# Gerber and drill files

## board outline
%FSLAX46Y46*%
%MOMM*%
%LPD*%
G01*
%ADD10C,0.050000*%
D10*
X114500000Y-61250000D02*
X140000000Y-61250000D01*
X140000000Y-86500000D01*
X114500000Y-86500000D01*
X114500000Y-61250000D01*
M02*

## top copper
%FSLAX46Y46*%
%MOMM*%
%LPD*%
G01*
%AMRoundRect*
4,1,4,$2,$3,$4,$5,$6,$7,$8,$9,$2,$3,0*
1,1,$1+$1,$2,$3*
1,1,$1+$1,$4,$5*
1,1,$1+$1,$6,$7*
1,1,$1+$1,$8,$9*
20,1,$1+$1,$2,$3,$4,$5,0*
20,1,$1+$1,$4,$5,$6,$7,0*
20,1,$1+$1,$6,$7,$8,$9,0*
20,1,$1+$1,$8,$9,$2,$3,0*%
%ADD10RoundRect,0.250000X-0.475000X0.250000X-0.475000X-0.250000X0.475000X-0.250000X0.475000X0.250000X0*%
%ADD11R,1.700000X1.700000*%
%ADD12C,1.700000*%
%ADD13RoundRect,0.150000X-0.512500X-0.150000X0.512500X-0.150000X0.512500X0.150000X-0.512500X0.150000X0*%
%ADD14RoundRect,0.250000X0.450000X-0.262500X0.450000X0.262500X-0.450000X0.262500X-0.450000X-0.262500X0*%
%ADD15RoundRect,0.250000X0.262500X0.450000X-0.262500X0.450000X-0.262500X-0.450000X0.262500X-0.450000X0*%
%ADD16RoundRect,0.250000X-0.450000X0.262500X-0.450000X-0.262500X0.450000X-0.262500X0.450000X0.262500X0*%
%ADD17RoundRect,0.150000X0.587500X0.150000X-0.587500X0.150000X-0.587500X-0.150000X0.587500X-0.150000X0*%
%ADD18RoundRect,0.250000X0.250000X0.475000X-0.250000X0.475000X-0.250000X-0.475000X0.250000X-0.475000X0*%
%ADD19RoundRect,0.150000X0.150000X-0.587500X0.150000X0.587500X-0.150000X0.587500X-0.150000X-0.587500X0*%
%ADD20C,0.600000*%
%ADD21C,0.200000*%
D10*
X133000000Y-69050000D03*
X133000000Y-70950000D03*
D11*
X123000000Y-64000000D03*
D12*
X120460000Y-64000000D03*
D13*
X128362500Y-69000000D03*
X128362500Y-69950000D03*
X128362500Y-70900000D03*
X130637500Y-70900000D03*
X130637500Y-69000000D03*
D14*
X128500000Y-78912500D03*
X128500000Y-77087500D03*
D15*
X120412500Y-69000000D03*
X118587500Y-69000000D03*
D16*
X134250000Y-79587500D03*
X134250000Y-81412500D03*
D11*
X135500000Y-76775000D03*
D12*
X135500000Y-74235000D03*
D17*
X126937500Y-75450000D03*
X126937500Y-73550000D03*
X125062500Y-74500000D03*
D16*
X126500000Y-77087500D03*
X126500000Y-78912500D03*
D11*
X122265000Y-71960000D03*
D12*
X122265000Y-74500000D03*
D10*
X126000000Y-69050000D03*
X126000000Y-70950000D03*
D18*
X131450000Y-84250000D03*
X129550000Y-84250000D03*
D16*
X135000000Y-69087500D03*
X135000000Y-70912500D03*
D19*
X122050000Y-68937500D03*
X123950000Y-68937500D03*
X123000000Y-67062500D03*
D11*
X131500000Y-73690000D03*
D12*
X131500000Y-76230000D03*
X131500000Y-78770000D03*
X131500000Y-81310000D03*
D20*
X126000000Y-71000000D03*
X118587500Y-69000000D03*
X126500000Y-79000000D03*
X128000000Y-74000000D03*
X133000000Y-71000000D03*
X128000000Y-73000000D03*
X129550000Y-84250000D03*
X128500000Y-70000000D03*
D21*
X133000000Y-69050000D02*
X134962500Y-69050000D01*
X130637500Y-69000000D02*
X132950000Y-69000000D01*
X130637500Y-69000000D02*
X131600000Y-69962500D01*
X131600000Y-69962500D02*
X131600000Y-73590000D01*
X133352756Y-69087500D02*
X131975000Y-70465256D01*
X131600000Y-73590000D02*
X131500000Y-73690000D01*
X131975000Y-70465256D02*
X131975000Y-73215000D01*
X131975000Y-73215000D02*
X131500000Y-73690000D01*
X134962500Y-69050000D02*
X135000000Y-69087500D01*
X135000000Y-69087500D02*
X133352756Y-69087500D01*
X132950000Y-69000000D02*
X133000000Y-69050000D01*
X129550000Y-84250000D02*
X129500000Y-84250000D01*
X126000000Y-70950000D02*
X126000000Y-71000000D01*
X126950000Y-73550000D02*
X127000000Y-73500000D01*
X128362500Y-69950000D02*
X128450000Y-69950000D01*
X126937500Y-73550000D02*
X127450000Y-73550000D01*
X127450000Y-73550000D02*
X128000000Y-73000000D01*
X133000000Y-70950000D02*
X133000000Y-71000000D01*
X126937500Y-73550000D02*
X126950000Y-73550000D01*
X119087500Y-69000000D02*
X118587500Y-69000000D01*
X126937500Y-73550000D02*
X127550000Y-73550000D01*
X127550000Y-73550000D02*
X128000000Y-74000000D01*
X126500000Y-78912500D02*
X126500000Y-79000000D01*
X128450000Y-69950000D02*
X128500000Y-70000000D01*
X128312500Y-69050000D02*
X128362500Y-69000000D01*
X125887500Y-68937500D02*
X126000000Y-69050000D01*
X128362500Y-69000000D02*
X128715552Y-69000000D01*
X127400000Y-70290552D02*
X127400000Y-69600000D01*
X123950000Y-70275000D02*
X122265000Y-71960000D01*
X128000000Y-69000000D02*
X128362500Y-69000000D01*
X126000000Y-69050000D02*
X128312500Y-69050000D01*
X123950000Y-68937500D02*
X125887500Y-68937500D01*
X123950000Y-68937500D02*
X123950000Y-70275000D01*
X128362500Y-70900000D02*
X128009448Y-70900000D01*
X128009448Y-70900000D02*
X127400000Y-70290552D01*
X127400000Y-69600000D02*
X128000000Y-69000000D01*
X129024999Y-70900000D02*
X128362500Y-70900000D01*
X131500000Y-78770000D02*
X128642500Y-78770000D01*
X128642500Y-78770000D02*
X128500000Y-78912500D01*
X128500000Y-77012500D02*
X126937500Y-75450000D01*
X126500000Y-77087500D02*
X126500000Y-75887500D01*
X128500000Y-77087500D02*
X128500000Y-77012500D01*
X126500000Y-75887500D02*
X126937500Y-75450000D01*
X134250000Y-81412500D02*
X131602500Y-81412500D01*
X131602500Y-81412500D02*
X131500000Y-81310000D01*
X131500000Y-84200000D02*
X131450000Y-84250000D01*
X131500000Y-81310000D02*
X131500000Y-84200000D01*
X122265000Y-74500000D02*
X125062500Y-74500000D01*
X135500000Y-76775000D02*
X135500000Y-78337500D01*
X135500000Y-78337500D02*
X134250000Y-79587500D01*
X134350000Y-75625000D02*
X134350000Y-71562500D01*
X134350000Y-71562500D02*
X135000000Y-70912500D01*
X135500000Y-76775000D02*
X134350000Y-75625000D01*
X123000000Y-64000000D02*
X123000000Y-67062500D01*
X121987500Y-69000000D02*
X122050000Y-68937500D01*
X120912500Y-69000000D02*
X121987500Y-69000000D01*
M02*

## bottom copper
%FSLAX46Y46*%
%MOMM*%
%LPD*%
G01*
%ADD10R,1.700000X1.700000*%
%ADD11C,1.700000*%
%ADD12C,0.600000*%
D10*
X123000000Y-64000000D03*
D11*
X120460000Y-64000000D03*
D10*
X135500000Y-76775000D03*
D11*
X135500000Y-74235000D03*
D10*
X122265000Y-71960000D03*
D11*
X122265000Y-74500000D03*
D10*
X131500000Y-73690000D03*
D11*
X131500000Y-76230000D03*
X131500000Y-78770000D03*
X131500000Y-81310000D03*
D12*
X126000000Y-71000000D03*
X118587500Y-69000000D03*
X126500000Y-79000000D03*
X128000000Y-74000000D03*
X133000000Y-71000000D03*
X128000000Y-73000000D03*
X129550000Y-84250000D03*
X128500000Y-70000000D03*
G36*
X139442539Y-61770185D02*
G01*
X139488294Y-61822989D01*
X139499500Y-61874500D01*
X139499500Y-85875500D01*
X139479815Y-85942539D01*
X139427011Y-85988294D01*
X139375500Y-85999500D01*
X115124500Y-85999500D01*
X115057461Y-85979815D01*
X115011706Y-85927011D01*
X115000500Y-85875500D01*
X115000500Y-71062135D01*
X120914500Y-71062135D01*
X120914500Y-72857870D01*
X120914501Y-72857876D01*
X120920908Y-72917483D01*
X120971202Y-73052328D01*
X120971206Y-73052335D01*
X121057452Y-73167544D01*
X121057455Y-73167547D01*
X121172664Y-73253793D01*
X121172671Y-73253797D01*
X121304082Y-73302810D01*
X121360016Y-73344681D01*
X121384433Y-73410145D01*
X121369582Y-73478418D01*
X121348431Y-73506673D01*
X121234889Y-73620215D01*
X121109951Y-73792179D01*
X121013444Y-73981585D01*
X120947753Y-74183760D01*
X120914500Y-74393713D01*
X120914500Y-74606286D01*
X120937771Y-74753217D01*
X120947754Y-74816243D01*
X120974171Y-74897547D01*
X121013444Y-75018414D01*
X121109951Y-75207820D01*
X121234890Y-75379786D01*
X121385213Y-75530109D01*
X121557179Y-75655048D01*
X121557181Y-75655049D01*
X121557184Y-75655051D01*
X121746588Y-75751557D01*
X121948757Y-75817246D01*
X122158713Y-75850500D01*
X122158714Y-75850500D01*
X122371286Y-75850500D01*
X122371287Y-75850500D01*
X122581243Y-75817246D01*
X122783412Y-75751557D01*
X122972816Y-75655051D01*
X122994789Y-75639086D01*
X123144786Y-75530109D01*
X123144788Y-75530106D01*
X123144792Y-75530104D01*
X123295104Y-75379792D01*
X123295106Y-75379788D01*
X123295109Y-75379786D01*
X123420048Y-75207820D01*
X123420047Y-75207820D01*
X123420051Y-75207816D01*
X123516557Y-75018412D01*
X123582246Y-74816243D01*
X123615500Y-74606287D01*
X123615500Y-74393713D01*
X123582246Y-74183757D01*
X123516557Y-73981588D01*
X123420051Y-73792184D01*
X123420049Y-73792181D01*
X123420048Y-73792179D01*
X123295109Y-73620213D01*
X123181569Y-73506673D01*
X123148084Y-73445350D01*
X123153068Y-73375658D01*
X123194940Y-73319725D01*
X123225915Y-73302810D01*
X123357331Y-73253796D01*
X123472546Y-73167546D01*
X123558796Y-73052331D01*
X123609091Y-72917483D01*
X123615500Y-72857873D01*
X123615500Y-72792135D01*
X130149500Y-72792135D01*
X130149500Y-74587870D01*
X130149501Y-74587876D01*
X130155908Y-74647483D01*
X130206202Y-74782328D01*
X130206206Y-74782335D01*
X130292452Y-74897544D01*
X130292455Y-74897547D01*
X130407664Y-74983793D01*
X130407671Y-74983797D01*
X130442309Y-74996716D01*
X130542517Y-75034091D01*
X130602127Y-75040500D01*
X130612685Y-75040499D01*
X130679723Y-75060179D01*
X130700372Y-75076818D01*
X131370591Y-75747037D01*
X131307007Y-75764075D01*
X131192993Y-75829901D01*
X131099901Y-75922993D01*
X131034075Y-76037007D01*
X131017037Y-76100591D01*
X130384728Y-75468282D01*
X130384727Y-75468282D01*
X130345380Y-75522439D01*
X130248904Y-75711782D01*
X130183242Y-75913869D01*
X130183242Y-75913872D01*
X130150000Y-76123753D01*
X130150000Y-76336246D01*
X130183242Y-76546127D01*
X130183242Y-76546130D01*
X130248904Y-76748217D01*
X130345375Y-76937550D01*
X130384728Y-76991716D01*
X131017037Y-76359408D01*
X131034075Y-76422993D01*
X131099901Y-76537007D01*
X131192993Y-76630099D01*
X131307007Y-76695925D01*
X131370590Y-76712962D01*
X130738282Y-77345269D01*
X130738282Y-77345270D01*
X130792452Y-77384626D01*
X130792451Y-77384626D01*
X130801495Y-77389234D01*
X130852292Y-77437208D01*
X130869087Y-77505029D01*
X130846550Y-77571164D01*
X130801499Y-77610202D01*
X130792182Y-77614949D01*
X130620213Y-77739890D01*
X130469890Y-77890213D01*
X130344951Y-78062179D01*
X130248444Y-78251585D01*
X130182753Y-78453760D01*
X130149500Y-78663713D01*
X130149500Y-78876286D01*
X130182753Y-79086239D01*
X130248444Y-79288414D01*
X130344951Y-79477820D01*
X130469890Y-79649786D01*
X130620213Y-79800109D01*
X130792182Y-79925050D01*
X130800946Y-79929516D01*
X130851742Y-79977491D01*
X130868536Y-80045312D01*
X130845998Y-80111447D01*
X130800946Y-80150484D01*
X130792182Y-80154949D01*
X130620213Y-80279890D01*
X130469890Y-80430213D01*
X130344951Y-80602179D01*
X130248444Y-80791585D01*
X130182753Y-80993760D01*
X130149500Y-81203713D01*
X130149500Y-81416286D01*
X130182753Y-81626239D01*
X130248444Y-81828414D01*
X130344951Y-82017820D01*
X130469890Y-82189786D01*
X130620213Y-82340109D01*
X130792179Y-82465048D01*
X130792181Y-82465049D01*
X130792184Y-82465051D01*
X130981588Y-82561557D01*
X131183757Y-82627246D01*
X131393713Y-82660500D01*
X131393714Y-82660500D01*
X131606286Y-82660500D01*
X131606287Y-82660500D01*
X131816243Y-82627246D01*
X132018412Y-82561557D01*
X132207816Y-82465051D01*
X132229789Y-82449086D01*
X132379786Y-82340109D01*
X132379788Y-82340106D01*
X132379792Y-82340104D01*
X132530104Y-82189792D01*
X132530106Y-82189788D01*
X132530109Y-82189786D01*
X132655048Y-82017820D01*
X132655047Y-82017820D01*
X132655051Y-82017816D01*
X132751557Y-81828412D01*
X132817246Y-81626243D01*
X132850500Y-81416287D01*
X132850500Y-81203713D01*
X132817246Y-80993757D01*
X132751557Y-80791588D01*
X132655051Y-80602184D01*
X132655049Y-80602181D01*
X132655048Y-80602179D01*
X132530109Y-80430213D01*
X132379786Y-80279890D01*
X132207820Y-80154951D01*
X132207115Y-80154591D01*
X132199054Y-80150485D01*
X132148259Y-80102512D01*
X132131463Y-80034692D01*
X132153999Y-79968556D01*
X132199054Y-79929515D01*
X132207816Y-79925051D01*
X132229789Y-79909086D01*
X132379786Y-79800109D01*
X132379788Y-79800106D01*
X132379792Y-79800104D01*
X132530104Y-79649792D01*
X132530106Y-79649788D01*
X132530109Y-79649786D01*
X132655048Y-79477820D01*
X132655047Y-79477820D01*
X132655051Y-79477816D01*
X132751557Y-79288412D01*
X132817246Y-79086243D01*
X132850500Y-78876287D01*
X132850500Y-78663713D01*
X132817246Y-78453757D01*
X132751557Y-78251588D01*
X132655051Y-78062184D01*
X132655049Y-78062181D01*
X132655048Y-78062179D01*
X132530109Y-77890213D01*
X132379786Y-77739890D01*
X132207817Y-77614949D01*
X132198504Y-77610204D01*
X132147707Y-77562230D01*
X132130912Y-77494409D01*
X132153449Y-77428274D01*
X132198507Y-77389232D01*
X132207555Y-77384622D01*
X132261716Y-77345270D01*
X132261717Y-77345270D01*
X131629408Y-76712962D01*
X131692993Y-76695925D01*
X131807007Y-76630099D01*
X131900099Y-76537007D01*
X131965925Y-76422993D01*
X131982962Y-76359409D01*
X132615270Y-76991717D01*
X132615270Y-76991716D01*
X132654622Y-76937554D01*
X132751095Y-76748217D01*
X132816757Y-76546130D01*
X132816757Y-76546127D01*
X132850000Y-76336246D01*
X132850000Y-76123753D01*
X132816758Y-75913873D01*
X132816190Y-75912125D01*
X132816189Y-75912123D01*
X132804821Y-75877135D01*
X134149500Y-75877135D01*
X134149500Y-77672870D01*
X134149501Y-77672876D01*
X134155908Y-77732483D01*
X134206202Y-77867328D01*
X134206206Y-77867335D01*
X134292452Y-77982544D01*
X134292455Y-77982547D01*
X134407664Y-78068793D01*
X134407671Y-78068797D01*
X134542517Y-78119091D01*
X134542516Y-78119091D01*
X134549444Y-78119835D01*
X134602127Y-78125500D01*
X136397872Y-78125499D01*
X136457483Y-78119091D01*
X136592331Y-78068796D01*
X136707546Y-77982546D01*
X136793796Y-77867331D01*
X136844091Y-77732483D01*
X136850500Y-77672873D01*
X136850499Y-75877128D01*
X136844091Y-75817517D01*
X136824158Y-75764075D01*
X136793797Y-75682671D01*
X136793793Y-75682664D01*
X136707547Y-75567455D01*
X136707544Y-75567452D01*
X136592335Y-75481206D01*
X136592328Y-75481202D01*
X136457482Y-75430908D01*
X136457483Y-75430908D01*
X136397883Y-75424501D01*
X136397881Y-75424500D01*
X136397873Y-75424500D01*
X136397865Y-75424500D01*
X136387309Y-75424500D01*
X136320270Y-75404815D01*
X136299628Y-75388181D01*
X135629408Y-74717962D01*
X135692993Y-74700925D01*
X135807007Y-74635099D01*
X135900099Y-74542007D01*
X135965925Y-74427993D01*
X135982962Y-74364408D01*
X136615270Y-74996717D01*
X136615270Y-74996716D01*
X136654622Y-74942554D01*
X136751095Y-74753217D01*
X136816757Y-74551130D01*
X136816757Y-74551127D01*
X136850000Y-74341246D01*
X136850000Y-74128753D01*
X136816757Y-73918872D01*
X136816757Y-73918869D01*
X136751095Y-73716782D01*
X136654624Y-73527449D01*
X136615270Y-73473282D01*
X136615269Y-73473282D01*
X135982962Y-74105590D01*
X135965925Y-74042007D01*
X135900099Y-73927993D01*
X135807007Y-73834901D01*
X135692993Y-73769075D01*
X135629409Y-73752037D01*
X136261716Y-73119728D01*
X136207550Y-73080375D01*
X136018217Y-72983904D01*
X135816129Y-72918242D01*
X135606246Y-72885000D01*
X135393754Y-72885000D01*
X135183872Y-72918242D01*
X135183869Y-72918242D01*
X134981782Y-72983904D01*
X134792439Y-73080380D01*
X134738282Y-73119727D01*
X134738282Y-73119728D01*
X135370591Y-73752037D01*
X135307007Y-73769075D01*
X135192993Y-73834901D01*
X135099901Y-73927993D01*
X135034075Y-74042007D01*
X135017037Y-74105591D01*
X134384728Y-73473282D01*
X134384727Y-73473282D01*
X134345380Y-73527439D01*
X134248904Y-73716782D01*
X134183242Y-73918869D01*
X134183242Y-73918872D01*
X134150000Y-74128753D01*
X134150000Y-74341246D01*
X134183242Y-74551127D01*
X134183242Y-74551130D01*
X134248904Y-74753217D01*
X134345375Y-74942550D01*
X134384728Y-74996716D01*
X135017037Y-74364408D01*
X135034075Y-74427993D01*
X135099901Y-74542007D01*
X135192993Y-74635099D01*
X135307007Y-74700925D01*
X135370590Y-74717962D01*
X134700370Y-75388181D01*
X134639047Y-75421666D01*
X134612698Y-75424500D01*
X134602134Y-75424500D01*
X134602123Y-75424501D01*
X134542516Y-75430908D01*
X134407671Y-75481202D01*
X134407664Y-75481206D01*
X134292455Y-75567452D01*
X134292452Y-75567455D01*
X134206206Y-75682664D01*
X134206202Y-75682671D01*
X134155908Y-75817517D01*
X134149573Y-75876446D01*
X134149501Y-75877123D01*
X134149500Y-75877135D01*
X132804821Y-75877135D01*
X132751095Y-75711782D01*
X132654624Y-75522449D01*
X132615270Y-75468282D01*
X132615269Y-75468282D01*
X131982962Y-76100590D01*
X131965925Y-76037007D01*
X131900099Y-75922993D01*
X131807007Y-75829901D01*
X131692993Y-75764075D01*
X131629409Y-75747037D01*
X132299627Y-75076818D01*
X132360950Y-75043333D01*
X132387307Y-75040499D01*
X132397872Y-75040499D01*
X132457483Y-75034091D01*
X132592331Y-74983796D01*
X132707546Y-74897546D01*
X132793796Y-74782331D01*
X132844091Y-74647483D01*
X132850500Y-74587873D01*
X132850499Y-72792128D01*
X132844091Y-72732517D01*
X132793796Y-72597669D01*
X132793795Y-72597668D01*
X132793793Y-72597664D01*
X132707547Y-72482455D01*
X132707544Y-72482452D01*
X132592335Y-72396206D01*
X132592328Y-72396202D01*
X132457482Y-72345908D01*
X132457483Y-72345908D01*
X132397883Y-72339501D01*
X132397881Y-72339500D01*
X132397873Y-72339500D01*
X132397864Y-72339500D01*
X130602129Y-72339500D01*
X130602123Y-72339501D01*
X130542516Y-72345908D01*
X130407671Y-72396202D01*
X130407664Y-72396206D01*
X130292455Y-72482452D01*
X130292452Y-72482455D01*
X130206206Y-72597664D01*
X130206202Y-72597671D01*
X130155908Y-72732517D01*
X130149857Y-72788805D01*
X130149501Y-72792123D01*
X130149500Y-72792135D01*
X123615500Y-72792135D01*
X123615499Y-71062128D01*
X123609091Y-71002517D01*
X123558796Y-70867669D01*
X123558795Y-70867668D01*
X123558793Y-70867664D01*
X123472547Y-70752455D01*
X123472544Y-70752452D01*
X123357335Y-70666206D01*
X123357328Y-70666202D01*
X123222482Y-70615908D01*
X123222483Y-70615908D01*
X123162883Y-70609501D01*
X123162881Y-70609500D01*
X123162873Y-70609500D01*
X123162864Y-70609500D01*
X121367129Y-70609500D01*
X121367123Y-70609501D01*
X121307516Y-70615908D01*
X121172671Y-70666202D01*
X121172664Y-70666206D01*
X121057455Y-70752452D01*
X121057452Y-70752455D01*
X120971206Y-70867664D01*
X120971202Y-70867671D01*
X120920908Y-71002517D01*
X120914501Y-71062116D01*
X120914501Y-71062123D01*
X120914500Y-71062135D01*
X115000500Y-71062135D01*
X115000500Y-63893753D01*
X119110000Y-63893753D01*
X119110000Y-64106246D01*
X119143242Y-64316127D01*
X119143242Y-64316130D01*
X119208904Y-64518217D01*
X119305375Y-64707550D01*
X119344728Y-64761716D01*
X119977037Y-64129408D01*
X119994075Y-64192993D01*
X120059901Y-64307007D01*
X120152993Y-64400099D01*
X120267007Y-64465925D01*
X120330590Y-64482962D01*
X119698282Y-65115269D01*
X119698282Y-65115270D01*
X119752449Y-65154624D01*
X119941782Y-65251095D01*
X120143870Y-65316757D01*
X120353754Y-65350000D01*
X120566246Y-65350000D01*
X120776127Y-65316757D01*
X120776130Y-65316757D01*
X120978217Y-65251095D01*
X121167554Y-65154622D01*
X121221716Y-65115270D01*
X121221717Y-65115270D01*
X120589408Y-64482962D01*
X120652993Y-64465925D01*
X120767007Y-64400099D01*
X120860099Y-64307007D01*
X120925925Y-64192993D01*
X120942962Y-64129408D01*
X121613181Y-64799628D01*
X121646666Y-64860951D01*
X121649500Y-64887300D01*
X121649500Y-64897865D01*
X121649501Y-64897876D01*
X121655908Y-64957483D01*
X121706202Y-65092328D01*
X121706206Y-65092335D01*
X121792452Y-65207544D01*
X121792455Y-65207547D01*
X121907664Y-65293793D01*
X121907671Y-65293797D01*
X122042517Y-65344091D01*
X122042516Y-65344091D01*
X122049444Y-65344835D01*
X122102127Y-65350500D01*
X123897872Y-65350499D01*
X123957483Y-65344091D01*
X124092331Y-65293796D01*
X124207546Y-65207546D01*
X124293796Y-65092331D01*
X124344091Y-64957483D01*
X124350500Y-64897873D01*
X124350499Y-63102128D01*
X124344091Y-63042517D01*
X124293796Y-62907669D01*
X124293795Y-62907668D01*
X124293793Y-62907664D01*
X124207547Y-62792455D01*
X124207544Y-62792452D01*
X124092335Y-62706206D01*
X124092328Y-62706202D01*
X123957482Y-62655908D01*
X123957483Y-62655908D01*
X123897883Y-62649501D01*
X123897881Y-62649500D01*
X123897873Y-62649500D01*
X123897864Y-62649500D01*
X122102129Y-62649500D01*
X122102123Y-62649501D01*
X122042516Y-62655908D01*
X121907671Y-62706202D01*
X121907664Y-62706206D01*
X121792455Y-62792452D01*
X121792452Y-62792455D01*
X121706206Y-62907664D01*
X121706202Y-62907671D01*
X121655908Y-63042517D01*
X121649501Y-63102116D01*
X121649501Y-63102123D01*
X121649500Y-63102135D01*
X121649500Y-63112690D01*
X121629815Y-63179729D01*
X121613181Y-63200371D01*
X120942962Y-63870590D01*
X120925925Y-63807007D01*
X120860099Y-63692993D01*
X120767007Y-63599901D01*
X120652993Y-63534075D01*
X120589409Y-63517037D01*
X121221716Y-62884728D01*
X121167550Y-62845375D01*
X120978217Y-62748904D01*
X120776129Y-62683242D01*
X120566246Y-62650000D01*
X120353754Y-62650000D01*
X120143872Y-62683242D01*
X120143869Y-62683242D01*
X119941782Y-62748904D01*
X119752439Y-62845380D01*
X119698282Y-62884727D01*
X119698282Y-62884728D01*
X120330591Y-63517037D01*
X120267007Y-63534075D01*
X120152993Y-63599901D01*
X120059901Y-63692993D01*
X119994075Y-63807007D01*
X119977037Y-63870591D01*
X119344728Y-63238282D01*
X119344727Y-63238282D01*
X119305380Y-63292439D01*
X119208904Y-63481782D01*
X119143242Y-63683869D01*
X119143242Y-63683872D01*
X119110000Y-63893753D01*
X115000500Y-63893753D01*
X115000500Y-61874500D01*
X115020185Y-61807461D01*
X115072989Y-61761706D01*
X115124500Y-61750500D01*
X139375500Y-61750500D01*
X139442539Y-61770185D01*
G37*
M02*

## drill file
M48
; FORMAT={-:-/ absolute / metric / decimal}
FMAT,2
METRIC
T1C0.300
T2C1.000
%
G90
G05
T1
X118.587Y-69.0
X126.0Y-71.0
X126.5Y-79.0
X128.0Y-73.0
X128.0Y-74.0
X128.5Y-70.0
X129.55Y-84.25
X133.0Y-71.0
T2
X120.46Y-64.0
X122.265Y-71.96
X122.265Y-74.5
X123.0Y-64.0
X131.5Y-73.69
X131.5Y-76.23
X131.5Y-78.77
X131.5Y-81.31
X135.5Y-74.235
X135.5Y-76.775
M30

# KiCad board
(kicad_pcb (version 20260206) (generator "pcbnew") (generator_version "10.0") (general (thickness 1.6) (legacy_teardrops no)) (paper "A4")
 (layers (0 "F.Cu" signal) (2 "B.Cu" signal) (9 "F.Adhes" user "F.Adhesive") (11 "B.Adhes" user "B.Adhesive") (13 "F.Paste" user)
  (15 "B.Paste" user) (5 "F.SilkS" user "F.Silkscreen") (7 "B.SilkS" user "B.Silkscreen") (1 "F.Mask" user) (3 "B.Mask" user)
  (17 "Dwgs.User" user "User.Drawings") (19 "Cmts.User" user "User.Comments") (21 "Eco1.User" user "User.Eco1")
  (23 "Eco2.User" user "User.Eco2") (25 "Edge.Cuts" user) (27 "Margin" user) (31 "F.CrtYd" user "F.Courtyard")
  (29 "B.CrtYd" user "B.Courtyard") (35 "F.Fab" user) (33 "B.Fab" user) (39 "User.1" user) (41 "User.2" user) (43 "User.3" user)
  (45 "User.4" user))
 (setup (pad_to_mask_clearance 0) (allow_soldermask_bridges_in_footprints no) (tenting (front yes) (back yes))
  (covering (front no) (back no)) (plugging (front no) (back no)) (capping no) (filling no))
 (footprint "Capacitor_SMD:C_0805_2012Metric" (layer "F.Cu") (at 133 70 -90)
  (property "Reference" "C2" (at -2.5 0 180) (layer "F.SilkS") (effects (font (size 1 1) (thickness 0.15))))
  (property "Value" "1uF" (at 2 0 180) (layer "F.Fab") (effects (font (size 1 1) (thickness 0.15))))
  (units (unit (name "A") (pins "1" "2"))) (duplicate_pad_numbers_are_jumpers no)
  (pad "1" smd roundrect (at -0.95 0 270) (size 1 1.45) (layers "F.Cu" "F.Mask" "F.Paste") (roundrect_rratio 0.25) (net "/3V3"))
  (pad "2" smd roundrect (at 0.95 0 270) (size 1 1.45) (layers "F.Cu" "F.Mask" "F.Paste") (roundrect_rratio 0.25) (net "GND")))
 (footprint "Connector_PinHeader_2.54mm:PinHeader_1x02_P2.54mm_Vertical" (layer "F.Cu") (at 123 64 -90)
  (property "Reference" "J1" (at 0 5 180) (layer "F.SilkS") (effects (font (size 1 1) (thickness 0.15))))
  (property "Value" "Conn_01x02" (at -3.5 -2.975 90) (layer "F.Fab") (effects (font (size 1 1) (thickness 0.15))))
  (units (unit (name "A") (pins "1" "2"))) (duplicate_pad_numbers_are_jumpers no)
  (pad "1" thru_hole rect (at 0 0 270) (size 1.7 1.7) (drill 1) (layers "*.Cu" "*.Mask") (remove_unused_layers no) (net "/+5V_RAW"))
  (pad "2" thru_hole circle (at 0 2.54 270) (size 1.7 1.7) (drill 1) (layers "*.Cu" "*.Mask") (remove_unused_layers no) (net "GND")))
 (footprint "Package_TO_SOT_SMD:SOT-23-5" (layer "F.Cu") (at 129.5 69.95)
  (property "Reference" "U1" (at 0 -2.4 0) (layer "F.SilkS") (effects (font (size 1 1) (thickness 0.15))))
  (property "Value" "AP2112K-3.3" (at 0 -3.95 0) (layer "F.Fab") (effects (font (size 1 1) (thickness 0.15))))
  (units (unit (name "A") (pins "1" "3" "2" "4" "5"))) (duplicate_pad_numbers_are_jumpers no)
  (pad "1" smd roundrect (at -1.1375 -0.95) (size 1.325 0.6) (layers "F.Cu" "F.Mask" "F.Paste") (roundrect_rratio 0.25) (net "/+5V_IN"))
  (pad "2" smd roundrect (at -1.1375 0) (size 1.325 0.6) (layers "F.Cu" "F.Mask" "F.Paste") (roundrect_rratio 0.25) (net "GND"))
  (pad "3" smd roundrect (at -1.1375 0.95) (size 1.325 0.6) (layers "F.Cu" "F.Mask" "F.Paste") (roundrect_rratio 0.25) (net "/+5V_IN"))
  (pad "4" smd roundrect (at 1.1375 0.95) (size 1.325 0.6) (layers "F.Cu" "F.Mask" "F.Paste") (roundrect_rratio 0.25)
   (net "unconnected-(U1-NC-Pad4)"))
  (pad "5" smd roundrect (at 1.1375 -0.95) (size 1.325 0.6) (layers "F.Cu" "F.Mask" "F.Paste") (roundrect_rratio 0.25) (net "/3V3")))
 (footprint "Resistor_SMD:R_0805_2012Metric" (layer "F.Cu") (at 128.5 78 90)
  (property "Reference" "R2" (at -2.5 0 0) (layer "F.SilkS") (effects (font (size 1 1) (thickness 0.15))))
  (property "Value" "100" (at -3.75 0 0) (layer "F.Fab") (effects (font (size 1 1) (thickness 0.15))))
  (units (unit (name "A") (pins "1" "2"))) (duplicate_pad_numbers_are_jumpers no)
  (pad "1" smd roundrect (at -0.9125 0 90) (size 1.025 1.4) (layers "F.Cu" "F.Mask" "F.Paste") (roundrect_rratio 0.243902) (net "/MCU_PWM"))
  (pad "2" smd roundrect (at 0.9125 0 90) (size 1.025 1.4) (layers "F.Cu" "F.Mask" "F.Paste") (roundrect_rratio 0.243902) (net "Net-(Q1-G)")))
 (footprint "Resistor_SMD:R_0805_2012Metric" (layer "F.Cu") (at 119.5 69 180)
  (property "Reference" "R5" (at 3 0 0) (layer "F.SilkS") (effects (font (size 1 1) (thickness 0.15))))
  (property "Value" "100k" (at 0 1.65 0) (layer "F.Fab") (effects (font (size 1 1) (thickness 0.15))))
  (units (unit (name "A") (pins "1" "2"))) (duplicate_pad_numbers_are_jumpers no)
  (pad "1" smd roundrect (at -0.9125 0 180) (size 1.025 1.4) (layers "F.Cu" "F.Mask" "F.Paste") (roundrect_rratio 0.243902)
   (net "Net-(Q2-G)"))
  (pad "2" smd roundrect (at 0.9125 0 180) (size 1.025 1.4) (layers "F.Cu" "F.Mask" "F.Paste") (roundrect_rratio 0.243902) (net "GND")))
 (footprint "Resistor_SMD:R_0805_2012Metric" (layer "F.Cu") (at 134.25 80.5 -90)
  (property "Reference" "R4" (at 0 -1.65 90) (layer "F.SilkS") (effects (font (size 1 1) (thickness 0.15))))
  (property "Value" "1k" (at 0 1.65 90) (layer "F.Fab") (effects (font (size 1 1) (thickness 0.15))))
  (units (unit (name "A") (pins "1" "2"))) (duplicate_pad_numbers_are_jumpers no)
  (pad "1" smd roundrect (at -0.9125 0 270) (size 1.025 1.4) (layers "F.Cu" "F.Mask" "F.Paste") (roundrect_rratio 0.243902)
   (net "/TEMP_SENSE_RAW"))
  (pad "2" smd roundrect (at 0.9125 0 270) (size 1.025 1.4) (layers "F.Cu" "F.Mask" "F.Paste") (roundrect_rratio 0.243902) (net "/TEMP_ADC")))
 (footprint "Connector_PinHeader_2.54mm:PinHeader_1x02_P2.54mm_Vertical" (layer "F.Cu") (at 135.5 76.775 180)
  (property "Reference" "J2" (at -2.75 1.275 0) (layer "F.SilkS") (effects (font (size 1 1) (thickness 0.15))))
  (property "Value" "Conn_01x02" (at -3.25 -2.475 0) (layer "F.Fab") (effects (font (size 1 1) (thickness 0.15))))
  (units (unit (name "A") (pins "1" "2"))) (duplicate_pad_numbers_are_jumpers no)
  (pad "1" thru_hole rect (at 0 0 180) (size 1.7 1.7) (drill 1) (layers "*.Cu" "*.Mask") (remove_unused_layers no) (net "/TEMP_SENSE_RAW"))
  (pad "2" thru_hole circle (at 0 2.54 180) (size 1.7 1.7) (drill 1) (layers "*.Cu" "*.Mask") (remove_unused_layers no) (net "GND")))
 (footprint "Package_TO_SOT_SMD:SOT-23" (layer "F.Cu") (at 126 74.5 180)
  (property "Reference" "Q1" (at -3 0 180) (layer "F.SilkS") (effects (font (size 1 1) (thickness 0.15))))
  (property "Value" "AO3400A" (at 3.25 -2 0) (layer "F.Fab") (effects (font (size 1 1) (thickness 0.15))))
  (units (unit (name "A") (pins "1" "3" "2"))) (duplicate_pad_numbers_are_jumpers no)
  (pad "1" smd roundrect (at -0.9375 -0.95 180) (size 1.475 0.6) (layers "F.Cu" "F.Mask" "F.Paste") (roundrect_rratio 0.25)
   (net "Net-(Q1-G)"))
  (pad "2" smd roundrect (at -0.9375 0.95 180) (size 1.475 0.6) (layers "F.Cu" "F.Mask" "F.Paste") (roundrect_rratio 0.25) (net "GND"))
  (pad "3" smd roundrect (at 0.9375 0 180) (size 1.475 0.6) (layers "F.Cu" "F.Mask" "F.Paste") (roundrect_rratio 0.25) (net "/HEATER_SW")))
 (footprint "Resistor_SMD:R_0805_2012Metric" (layer "F.Cu") (at 126.5 78 -90)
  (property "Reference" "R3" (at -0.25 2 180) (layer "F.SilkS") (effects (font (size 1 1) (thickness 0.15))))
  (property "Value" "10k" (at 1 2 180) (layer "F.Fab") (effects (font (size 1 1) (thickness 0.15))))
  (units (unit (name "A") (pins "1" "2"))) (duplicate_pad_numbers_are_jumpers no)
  (pad "1" smd roundrect (at -0.9125 0 270) (size 1.025 1.4) (layers "F.Cu" "F.Mask" "F.Paste") (roundrect_rratio 0.243902)
   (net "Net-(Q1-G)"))
  (pad "2" smd roundrect (at 0.9125 0 270) (size 1.025 1.4) (layers "F.Cu" "F.Mask" "F.Paste") (roundrect_rratio 0.243902) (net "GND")))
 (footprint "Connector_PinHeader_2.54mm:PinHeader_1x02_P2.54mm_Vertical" (layer "F.Cu") (at 122.265 71.96)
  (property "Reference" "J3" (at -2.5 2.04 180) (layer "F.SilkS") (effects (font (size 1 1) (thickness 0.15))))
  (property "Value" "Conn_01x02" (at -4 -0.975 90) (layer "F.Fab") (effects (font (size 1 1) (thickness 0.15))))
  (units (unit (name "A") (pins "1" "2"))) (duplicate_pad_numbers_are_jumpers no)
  (pad "1" thru_hole rect (at 0 0) (size 1.7 1.7) (drill 1) (layers "*.Cu" "*.Mask") (remove_unused_layers no) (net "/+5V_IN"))
  (pad "2" thru_hole circle (at 0 2.54) (size 1.7 1.7) (drill 1) (layers "*.Cu" "*.Mask") (remove_unused_layers no) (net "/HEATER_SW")))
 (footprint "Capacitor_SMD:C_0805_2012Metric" (layer "F.Cu") (at 126 70 -90)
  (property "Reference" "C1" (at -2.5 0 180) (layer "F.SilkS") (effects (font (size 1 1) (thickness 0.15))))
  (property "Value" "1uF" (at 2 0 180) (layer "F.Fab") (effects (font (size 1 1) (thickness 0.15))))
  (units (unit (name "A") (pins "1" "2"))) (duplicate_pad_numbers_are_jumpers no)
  (pad "1" smd roundrect (at -0.95 0 270) (size 1 1.45) (layers "F.Cu" "F.Mask" "F.Paste") (roundrect_rratio 0.25) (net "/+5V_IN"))
  (pad "2" smd roundrect (at 0.95 0 270) (size 1 1.45) (layers "F.Cu" "F.Mask" "F.Paste") (roundrect_rratio 0.25) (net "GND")))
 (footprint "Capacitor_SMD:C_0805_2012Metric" (layer "F.Cu") (at 130.5 84.25 180)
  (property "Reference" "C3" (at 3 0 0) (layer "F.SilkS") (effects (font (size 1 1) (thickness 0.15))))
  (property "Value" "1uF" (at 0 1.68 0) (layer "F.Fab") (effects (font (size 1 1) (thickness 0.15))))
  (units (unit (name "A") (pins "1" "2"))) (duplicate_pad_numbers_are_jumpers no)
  (pad "1" smd roundrect (at -0.95 0 180) (size 1 1.45) (layers "F.Cu" "F.Mask" "F.Paste") (roundrect_rratio 0.25) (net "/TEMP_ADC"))
  (pad "2" smd roundrect (at 0.95 0 180) (size 1 1.45) (layers "F.Cu" "F.Mask" "F.Paste") (roundrect_rratio 0.25) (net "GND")))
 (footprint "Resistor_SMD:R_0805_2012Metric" (layer "F.Cu") (at 135 70 -90)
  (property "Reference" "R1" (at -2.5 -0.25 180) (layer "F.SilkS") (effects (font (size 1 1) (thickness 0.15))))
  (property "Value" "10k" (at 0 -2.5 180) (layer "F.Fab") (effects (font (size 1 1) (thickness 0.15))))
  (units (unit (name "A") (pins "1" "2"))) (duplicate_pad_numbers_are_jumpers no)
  (pad "1" smd roundrect (at -0.9125 0 270) (size 1.025 1.4) (layers "F.Cu" "F.Mask" "F.Paste") (roundrect_rratio 0.243902) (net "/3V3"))
  (pad "2" smd roundrect (at 0.9125 0 270) (size 1.025 1.4) (layers "F.Cu" "F.Mask" "F.Paste") (roundrect_rratio 0.243902)
   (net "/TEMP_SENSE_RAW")))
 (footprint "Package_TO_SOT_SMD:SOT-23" (layer "F.Cu") (at 123 68 90)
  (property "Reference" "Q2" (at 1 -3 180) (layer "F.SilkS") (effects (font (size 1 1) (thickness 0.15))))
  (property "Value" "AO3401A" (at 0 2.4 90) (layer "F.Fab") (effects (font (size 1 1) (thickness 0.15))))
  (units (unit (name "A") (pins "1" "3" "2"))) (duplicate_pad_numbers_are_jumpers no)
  (pad "1" smd roundrect (at -0.9375 -0.95 90) (size 1.475 0.6) (layers "F.Cu" "F.Mask" "F.Paste") (roundrect_rratio 0.25)
   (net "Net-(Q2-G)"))
  (pad "2" smd roundrect (at -0.9375 0.95 90) (size 1.475 0.6) (layers "F.Cu" "F.Mask" "F.Paste") (roundrect_rratio 0.25) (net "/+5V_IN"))
  (pad "3" smd roundrect (at 0.9375 0 90) (size 1.475 0.6) (layers "F.Cu" "F.Mask" "F.Paste") (roundrect_rratio 0.25) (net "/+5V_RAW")))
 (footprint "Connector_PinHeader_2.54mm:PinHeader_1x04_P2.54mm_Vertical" (layer "F.Cu") (at 131.5 73.69)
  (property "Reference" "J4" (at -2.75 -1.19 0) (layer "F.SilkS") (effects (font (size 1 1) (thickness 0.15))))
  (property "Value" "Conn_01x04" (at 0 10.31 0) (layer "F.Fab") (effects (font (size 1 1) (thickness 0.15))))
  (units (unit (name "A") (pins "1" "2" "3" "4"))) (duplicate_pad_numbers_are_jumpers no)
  (pad "1" thru_hole rect (at 0 0) (size 1.7 1.7) (drill 1) (layers "*.Cu" "*.Mask") (remove_unused_layers no) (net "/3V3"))
  (pad "2" thru_hole circle (at 0 2.54) (size 1.7 1.7) (drill 1) (layers "*.Cu" "*.Mask") (remove_unused_layers no) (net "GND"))
  (pad "3" thru_hole circle (at 0 5.08) (size 1.7 1.7) (drill 1) (layers "*.Cu" "*.Mask") (remove_unused_layers no) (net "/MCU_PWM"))
  (pad "4" thru_hole circle (at 0 7.62) (size 1.7 1.7) (drill 1) (layers "*.Cu" "*.Mask") (remove_unused_layers no) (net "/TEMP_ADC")))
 (gr_rect (start 114.5 61.25) (end 140 86.5) (stroke (width 0.05) (type default)) (fill no) (layer "Edge.Cuts"))
 (segment (start 133 69.05) (end 134.9625 69.05) (width 0.2) (layer "F.Cu") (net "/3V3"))
 (segment (start 130.6375 69) (end 132.95 69) (width 0.2) (layer "F.Cu") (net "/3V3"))
 (segment (start 130.6375 69) (end 131.6 69.9625) (width 0.2) (layer "F.Cu") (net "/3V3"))
 (segment (start 131.6 69.9625) (end 131.6 73.59) (width 0.2) (layer "F.Cu") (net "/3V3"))
 (segment (start 133.352756 69.0875) (end 131.975 70.465256) (width 0.2) (layer "F.Cu") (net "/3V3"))
 (segment (start 131.6 73.59) (end 131.5 73.69) (width 0.2) (layer "F.Cu") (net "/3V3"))
 (segment (start 131.975 70.465256) (end 131.975 73.215) (width 0.2) (layer "F.Cu") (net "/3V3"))
 (segment (start 131.975 73.215) (end 131.5 73.69) (width 0.2) (layer "F.Cu") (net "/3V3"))
 (segment (start 134.9625 69.05) (end 135 69.0875) (width 0.2) (layer "F.Cu") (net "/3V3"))
 (segment (start 135 69.0875) (end 133.352756 69.0875) (width 0.2) (layer "F.Cu") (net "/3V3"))
 (segment (start 132.95 69) (end 133 69.05) (width 0.2) (layer "F.Cu") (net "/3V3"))
 (segment (start 129.55 84.25) (end 129.5 84.25) (width 0.2) (layer "F.Cu") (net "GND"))
 (segment (start 126 70.95) (end 126 71) (width 0.2) (layer "F.Cu") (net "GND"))
 (segment (start 126.95 73.55) (end 127 73.5) (width 0.2) (layer "F.Cu") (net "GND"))
 (segment (start 128.3625 69.95) (end 128.45 69.95) (width 0.2) (layer "F.Cu") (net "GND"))
 (segment (start 126.9375 73.55) (end 127.45 73.55) (width 0.2) (layer "F.Cu") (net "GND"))
 (segment (start 127.45 73.55) (end 128 73) (width 0.2) (layer "F.Cu") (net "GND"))
 (segment (start 133 70.95) (end 133 71) (width 0.2) (layer "F.Cu") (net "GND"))
 (segment (start 126.9375 73.55) (end 126.95 73.55) (width 0.2) (layer "F.Cu") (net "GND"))
 (segment (start 119.0875 69) (end 118.5875 69) (width 0.2) (layer "F.Cu") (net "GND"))
 (segment (start 126.9375 73.55) (end 127.55 73.55) (width 0.2) (layer "F.Cu") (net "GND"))
 (segment (start 127.55 73.55) (end 128 74) (width 0.2) (layer "F.Cu") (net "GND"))
 (segment (start 126.5 78.9125) (end 126.5 79) (width 0.2) (layer "F.Cu") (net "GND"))
 (segment (start 128.45 69.95) (end 128.5 70) (width 0.2) (layer "F.Cu") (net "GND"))
 (via (at 126 71) (size 0.6) (drill 0.3) (layers "F.Cu" "B.Cu") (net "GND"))
 (via (at 118.5875 69) (size 0.6) (drill 0.3) (layers "F.Cu" "B.Cu") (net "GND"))
 (via (at 126.5 79) (size 0.6) (drill 0.3) (layers "F.Cu" "B.Cu") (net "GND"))
 (via (at 128 74) (size 0.6) (drill 0.3) (layers "F.Cu" "B.Cu") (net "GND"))
 (via (at 133 71) (size 0.6) (drill 0.3) (layers "F.Cu" "B.Cu") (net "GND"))
 (via (at 128 73) (size 0.6) (drill 0.3) (layers "F.Cu" "B.Cu") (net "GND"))
 (via (at 129.55 84.25) (size 0.6) (drill 0.3) (layers "F.Cu" "B.Cu") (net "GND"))
 (via (at 128.5 70) (size 0.6) (drill 0.3) (layers "F.Cu" "B.Cu") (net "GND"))
 (segment (start 128.3125 69.05) (end 128.3625 69) (width 0.2) (layer "F.Cu") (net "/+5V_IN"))
 (segment (start 125.8875 68.9375) (end 126 69.05) (width 0.2) (layer "F.Cu") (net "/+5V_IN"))
 (segment (start 128.3625 69) (end 128.715552 69) (width 0.2) (layer "F.Cu") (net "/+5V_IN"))
 (segment (start 127.4 70.290552) (end 127.4 69.6) (width 0.2) (layer "F.Cu") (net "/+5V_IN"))
 (segment (start 123.95 70.275) (end 122.265 71.96) (width 0.2) (layer "F.Cu") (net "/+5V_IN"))
 (segment (start 128 69) (end 128.3625 69) (width 0.2) (layer "F.Cu") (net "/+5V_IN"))
 (segment (start 126 69.05) (end 128.3125 69.05) (width 0.2) (layer "F.Cu") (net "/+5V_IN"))
 (segment (start 123.95 68.9375) (end 125.8875 68.9375) (width 0.2) (layer "F.Cu") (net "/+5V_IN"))
 (segment (start 123.95 68.9375) (end 123.95 70.275) (width 0.2) (layer "F.Cu") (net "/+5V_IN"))
 (segment (start 128.3625 70.9) (end 128.009448 70.9) (width 0.2) (layer "F.Cu") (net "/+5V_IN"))
 (segment (start 128.009448 70.9) (end 127.4 70.290552) (width 0.2) (layer "F.Cu") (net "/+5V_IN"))
 (segment (start 127.4 69.6) (end 128 69) (width 0.2) (layer "F.Cu") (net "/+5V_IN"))
 (segment (start 129.024999 70.9) (end 128.3625 70.9) (width 0.2) (layer "F.Cu") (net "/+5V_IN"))
 (segment (start 131.5 78.77) (end 128.6425 78.77) (width 0.2) (layer "F.Cu") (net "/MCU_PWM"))
 (segment (start 128.6425 78.77) (end 128.5 78.9125) (width 0.2) (layer "F.Cu") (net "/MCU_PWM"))
 (segment (start 128.5 77.0125) (end 126.9375 75.45) (width 0.2) (layer "F.Cu") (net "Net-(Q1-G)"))
 (segment (start 126.5 77.0875) (end 126.5 75.8875) (width 0.2) (layer "F.Cu") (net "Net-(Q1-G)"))
 (segment (start 128.5 77.0875) (end 128.5 77.0125) (width 0.2) (layer "F.Cu") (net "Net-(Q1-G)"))
 (segment (start 126.5 75.8875) (end 126.9375 75.45) (width 0.2) (layer "F.Cu") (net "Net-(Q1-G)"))
 (segment (start 134.25 81.4125) (end 131.6025 81.4125) (width 0.2) (layer "F.Cu") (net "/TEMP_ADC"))
 (segment (start 131.6025 81.4125) (end 131.5 81.31) (width 0.2) (layer "F.Cu") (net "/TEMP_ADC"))
 (segment (start 131.5 84.2) (end 131.45 84.25) (width 0.2) (layer "F.Cu") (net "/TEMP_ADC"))
 (segment (start 131.5 81.31) (end 131.5 84.2) (width 0.2) (layer "F.Cu") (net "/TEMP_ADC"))
 (segment (start 122.265 74.5) (end 125.0625 74.5) (width 0.2) (layer "F.Cu") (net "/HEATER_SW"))
 (segment (start 135.5 76.775) (end 135.5 78.3375) (width 0.2) (layer "F.Cu") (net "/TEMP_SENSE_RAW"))
 (segment (start 135.5 78.3375) (end 134.25 79.5875) (width 0.2) (layer "F.Cu") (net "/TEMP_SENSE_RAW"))
 (segment (start 134.35 75.625) (end 134.35 71.5625) (width 0.2) (layer "F.Cu") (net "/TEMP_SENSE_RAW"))
 (segment (start 134.35 71.5625) (end 135 70.9125) (width 0.2) (layer "F.Cu") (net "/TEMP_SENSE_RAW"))
 (segment (start 135.5 76.775) (end 134.35 75.625) (width 0.2) (layer "F.Cu") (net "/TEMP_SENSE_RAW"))
 (segment (start 123 64) (end 123 67.0625) (width 0.2) (layer "F.Cu") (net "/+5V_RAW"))
 (segment (start 121.9875 69) (end 122.05 68.9375) (width 0.2) (layer "F.Cu") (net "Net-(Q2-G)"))
 (segment (start 120.9125 69) (end 121.9875 69) (width 0.2) (layer "F.Cu") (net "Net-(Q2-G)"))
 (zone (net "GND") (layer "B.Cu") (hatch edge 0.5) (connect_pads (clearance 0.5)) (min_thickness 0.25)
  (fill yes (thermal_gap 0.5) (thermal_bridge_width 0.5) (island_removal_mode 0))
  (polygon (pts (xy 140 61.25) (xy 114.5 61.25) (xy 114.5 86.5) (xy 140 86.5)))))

